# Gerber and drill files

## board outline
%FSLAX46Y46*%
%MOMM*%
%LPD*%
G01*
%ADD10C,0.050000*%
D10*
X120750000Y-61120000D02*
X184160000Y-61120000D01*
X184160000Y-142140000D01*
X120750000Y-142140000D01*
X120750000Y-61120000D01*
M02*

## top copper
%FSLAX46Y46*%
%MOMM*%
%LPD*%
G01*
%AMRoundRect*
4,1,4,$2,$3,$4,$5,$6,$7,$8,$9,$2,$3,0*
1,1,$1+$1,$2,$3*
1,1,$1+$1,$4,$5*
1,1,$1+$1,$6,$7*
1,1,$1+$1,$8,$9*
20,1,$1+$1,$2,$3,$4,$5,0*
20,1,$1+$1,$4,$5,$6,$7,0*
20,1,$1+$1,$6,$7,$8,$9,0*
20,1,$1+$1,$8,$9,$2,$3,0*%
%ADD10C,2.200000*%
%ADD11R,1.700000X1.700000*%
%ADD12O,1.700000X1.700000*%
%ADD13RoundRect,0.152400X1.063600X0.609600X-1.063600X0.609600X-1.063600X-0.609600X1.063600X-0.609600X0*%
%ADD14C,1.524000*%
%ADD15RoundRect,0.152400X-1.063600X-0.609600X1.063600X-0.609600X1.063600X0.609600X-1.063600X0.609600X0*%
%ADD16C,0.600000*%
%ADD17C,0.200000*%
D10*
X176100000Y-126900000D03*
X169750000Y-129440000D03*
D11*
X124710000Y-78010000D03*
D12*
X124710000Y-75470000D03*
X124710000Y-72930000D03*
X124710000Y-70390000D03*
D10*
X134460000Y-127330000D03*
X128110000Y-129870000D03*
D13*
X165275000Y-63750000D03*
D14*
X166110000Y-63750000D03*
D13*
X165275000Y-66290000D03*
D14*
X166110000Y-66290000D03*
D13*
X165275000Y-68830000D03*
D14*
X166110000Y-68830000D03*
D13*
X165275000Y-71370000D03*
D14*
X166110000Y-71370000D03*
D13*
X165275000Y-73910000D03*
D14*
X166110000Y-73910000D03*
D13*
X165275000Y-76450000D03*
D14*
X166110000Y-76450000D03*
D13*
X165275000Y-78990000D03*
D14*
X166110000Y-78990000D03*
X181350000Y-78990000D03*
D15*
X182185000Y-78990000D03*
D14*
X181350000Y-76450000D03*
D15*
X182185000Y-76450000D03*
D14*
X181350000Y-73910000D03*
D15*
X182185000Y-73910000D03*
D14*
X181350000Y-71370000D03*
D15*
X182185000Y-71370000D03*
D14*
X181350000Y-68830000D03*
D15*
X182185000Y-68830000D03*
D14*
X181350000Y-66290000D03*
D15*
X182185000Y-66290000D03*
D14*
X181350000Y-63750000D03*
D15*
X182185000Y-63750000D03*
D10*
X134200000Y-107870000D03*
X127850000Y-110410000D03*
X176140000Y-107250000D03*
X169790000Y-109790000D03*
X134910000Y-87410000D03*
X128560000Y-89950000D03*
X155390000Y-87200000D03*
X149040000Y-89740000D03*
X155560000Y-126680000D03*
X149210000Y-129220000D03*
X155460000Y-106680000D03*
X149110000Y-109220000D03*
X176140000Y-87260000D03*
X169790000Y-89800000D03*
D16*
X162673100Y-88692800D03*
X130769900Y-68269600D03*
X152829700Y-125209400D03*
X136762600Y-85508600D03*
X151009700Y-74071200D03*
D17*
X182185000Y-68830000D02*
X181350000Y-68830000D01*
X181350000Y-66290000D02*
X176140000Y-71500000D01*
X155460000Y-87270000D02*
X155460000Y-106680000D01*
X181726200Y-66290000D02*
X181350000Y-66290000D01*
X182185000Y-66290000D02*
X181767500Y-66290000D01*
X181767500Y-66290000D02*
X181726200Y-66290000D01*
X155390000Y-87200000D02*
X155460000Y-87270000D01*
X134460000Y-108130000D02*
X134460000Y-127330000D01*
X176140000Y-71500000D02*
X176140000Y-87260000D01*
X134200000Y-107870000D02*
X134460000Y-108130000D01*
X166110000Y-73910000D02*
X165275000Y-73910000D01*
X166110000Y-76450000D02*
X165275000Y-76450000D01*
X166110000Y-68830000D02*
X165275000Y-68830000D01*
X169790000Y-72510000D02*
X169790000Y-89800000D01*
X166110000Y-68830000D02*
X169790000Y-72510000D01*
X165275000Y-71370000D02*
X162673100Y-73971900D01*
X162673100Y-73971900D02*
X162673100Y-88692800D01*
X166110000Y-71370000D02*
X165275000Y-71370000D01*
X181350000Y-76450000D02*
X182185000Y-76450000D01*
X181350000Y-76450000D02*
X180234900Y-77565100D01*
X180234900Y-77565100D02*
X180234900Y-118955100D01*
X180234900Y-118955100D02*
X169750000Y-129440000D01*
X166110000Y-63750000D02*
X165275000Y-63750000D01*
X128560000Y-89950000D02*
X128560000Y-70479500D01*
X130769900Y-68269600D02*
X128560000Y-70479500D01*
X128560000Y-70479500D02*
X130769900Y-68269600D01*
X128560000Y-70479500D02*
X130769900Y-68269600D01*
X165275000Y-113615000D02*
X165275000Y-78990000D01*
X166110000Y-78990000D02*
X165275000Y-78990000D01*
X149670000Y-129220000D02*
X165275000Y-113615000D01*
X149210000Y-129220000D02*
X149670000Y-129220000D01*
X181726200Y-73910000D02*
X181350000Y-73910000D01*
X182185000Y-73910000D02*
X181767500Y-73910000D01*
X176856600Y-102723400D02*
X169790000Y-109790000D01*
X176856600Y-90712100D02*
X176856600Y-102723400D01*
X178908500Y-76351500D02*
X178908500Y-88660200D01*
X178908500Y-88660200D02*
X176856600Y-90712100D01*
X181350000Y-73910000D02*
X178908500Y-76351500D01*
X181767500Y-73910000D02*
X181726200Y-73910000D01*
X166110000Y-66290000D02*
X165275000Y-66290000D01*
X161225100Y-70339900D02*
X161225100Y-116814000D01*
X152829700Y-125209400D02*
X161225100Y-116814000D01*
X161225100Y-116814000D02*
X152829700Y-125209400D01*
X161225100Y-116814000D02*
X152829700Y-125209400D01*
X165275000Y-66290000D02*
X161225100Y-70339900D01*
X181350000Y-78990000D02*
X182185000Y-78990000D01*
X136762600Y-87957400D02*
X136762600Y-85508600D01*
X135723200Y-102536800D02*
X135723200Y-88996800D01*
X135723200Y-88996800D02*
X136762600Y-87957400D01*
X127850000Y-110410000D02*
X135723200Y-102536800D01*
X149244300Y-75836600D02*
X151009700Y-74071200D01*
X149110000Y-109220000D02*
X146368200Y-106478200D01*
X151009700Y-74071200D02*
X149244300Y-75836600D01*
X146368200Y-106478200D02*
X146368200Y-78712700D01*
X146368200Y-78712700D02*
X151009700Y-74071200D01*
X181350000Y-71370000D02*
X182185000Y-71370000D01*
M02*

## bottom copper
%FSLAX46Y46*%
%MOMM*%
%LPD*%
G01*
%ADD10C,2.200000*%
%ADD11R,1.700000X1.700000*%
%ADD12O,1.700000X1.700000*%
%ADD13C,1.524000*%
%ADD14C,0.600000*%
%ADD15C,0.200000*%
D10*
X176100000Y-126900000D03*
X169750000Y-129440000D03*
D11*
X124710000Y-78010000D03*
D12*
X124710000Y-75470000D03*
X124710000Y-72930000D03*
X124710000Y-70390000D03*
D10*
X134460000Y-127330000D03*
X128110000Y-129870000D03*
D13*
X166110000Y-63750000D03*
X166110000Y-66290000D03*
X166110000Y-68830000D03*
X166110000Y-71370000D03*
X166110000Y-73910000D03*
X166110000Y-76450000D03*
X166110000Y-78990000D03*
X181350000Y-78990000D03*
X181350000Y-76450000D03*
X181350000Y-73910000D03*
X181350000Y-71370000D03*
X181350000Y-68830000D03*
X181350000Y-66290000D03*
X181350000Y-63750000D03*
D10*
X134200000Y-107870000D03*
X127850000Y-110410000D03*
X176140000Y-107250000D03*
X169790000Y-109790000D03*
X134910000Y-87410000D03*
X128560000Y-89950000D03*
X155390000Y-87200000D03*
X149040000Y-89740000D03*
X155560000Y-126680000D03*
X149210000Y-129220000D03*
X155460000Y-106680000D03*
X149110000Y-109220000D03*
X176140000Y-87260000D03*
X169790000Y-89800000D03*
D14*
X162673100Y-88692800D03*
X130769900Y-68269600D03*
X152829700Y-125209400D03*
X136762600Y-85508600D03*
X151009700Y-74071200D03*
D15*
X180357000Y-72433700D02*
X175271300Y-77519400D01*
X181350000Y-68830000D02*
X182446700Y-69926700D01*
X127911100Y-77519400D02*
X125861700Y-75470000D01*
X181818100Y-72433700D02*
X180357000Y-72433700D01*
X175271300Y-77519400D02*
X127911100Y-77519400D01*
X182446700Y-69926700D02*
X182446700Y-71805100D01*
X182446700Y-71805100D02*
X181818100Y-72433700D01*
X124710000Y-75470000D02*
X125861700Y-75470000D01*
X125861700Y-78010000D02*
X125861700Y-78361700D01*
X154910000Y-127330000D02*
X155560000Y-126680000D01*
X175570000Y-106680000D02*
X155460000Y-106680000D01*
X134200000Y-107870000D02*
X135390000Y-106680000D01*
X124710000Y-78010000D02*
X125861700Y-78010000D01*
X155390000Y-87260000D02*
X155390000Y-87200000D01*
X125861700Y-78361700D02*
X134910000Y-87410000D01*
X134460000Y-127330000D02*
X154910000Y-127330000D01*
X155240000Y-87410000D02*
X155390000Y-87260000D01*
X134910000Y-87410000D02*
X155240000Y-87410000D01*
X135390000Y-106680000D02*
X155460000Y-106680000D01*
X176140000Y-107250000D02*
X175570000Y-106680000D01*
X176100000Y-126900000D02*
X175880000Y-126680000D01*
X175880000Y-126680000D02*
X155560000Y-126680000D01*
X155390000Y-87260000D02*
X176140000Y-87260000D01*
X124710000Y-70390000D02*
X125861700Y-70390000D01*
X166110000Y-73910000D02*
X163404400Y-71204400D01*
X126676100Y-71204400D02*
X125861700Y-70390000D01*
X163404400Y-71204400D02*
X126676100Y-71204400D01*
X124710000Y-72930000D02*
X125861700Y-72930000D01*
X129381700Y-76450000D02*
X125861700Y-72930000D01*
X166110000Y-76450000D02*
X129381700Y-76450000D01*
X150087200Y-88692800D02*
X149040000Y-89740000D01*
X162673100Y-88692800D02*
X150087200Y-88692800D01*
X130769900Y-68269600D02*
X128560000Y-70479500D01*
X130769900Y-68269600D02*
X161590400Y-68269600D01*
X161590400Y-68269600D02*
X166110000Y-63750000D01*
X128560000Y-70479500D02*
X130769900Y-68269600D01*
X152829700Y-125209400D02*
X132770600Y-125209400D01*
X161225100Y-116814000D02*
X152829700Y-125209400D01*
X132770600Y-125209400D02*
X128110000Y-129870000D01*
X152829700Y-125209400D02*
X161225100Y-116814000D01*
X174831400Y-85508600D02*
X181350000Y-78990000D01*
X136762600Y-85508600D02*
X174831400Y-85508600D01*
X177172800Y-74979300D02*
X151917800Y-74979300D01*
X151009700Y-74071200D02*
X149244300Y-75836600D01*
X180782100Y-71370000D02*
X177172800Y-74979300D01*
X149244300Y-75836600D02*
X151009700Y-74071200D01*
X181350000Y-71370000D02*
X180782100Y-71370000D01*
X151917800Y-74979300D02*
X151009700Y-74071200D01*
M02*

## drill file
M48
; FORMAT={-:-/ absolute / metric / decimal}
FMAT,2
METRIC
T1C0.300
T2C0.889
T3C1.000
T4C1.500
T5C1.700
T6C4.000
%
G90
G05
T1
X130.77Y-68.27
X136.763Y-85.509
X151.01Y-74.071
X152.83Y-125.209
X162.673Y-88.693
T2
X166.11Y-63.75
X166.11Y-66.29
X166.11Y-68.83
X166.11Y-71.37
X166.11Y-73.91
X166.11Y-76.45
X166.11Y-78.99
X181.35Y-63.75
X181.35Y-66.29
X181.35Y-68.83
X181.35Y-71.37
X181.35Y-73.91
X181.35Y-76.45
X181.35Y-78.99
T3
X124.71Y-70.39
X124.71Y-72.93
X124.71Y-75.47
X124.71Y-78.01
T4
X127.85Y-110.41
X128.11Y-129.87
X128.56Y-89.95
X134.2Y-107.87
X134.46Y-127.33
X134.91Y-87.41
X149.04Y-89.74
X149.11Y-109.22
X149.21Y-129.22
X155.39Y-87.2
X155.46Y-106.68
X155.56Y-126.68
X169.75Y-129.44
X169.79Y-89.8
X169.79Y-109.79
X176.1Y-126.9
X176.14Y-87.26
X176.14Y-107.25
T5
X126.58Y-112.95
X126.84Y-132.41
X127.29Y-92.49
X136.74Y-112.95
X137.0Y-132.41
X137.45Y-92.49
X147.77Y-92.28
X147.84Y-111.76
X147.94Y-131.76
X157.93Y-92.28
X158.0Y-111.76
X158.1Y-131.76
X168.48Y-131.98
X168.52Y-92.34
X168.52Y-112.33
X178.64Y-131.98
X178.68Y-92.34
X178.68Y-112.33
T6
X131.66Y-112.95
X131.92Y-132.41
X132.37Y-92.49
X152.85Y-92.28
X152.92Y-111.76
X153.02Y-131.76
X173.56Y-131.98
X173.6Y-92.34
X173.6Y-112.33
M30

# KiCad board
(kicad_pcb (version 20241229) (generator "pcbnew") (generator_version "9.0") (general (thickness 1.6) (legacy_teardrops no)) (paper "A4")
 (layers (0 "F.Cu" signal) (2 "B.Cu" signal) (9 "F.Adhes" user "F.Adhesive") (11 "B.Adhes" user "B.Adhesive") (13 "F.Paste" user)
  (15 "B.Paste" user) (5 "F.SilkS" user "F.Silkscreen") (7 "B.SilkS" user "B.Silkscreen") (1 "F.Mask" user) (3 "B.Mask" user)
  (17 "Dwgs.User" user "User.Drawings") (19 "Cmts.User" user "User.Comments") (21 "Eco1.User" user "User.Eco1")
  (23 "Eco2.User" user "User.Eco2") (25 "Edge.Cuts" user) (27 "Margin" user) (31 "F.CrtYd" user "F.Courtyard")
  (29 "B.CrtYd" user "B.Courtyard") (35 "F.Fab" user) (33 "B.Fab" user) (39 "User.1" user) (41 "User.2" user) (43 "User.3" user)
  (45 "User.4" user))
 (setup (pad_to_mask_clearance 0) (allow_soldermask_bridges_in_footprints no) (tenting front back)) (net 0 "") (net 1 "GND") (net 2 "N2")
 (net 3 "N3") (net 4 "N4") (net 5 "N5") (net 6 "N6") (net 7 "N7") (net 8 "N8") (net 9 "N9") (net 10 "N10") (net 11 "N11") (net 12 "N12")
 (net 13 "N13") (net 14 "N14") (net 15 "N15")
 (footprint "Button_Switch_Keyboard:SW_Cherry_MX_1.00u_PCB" (layer "F.Cu") (at 176.1 126.9)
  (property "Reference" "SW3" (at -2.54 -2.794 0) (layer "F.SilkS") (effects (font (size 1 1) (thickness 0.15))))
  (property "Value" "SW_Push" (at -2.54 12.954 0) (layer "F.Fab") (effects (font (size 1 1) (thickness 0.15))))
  (pad "" np_thru_hole circle (at -7.62 5.08) (size 1.7 1.7) (drill 1.7) (layers "*.Cu" "*.Mask"))
  (pad "" np_thru_hole circle (at -2.54 5.08) (size 4 4) (drill 4) (layers "*.Cu" "*.Mask"))
  (pad "" np_thru_hole circle (at 2.54 5.08) (size 1.7 1.7) (drill 1.7) (layers "*.Cu" "*.Mask"))
  (pad "1" thru_hole circle (at 0 0) (size 2.2 2.2) (drill 1.5) (layers "*.Cu" "*.Mask") (remove_unused_layers no) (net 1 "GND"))
  (pad "2" thru_hole circle (at -6.35 2.54) (size 2.2 2.2) (drill 1.5) (layers "*.Cu" "*.Mask") (remove_unused_layers no) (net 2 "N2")))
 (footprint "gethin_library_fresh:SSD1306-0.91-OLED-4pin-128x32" (layer "F.Cu") (at 161.21 80.2 180)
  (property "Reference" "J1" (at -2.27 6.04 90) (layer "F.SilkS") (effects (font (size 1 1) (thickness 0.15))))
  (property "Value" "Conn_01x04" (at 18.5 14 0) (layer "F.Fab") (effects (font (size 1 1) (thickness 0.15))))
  (pad "1" thru_hole rect (at 36.5 2.19 180) (size 1.7 1.7) (drill 1) (layers "*.Cu" "*.Mask") (remove_unused_layers no) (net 1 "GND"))
  (pad "2" thru_hole oval (at 36.5 4.73 180) (size 1.7 1.7) (drill 1) (layers "*.Cu" "*.Mask") (remove_unused_layers no) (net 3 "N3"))
  (pad "3" thru_hole oval (at 36.5 7.27 180) (size 1.7 1.7) (drill 1) (layers "*.Cu" "*.Mask") (remove_unused_layers no) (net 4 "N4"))
  (pad "4" thru_hole oval (at 36.5 9.81 180) (size 1.7 1.7) (drill 1) (layers "*.Cu" "*.Mask") (remove_unused_layers no) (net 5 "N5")))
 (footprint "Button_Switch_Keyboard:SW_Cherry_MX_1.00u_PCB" (layer "F.Cu") (at 134.46 127.33)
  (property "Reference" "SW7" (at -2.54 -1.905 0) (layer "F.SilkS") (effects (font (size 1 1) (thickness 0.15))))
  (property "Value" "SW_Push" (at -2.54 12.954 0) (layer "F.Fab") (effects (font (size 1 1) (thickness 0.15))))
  (pad "" np_thru_hole circle (at -7.62 5.08) (size 1.7 1.7) (drill 1.7) (layers "*.Cu" "*.Mask"))
  (pad "" np_thru_hole circle (at -2.54 5.08) (size 4 4) (drill 4) (layers "*.Cu" "*.Mask"))
  (pad "" np_thru_hole circle (at 2.54 5.08) (size 1.7 1.7) (drill 1.7) (layers "*.Cu" "*.Mask"))
  (pad "1" thru_hole circle (at 0 0) (size 2.2 2.2) (drill 1.5) (layers "*.Cu" "*.Mask") (remove_unused_layers no) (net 1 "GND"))
  (pad "2" thru_hole circle (at -6.35 2.54) (size 2.2 2.2) (drill 1.5) (layers "*.Cu" "*.Mask") (remove_unused_layers no) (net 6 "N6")))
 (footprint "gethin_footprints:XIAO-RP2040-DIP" (layer "F.Cu") (at 173.73 71.37)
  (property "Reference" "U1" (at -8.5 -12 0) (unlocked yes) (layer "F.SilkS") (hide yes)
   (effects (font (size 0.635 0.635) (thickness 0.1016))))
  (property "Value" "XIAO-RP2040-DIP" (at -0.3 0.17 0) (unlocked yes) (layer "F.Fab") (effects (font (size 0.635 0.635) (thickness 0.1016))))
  (pad "1" smd roundrect (at -8.455 -7.62 180) (size 2.432 1.524) (layers "F.Cu" "F.Mask") (roundrect_rratio 0.1) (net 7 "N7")
   (thermal_bridge_angle 45))
  (pad "1" thru_hole circle (at -7.62 -7.62 180) (size 1.524 1.524) (drill 0.889) (layers "*.Cu" "*.Mask") (remove_unused_layers no)
   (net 7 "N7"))
  (pad "2" smd roundrect (at -8.455 -5.08 180) (size 2.432 1.524) (layers "F.Cu" "F.Mask") (roundrect_rratio 0.1) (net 6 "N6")
   (thermal_bridge_angle 45))
  (pad "2" thru_hole circle (at -7.62 -5.08 180) (size 1.524 1.524) (drill 0.889) (layers "*.Cu" "*.Mask") (remove_unused_layers no)
   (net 6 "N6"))
  (pad "3" smd roundrect (at -8.455 -2.54 180) (size 2.432 1.524) (layers "F.Cu" "F.Mask") (roundrect_rratio 0.1) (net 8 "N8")
   (thermal_bridge_angle 45))
  (pad "3" thru_hole circle (at -7.62 -2.54 180) (size 1.524 1.524) (drill 0.889) (layers "*.Cu" "*.Mask") (remove_unused_layers no)
   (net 8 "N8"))
  (pad "4" smd roundrect (at -8.455 0 180) (size 2.432 1.524) (layers "F.Cu" "F.Mask") (roundrect_rratio 0.1) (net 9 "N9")
   (thermal_bridge_angle 45))
  (pad "4" thru_hole circle (at -7.62 0 180) (size 1.524 1.524) (drill 0.889) (layers "*.Cu" "*.Mask") (remove_unused_layers no)
   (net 9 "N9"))
  (pad "5" smd roundrect (at -8.455 2.54 180) (size 2.432 1.524) (layers "F.Cu" "F.Mask") (roundrect_rratio 0.1) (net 5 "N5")
   (thermal_bridge_angle 45))
  (pad "5" thru_hole circle (at -7.62 2.54 180) (size 1.524 1.524) (drill 0.889) (layers "*.Cu" "*.Mask") (remove_unused_layers no)
   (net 5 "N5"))
  (pad "6" smd roundrect (at -8.455 5.08 180) (size 2.432 1.524) (layers "F.Cu" "F.Mask") (roundrect_rratio 0.1) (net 4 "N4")
   (thermal_bridge_angle 45))
  (pad "6" thru_hole circle (at -7.62 5.08 180) (size 1.524 1.524) (drill 0.889) (layers "*.Cu" "*.Mask") (remove_unused_layers no)
   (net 4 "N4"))
  (pad "7" smd roundrect (at -8.455 7.62 180) (size 2.432 1.524) (layers "F.Cu" "F.Mask") (roundrect_rratio 0.1) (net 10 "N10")
   (thermal_bridge_angle 45))
  (pad "7" thru_hole circle (at -7.62 7.62 180) (size 1.524 1.524) (drill 0.889) (layers "*.Cu" "*.Mask") (remove_unused_layers no)
   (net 10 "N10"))
  (pad "8" thru_hole circle (at 7.62 7.62) (size 1.524 1.524) (drill 0.889) (layers "*.Cu" "*.Mask") (remove_unused_layers no)
   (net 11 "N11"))
  (pad "8" smd roundrect (at 8.455 7.62) (size 2.432 1.524) (layers "F.Cu" "F.Mask") (roundrect_rratio 0.1) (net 11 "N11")
   (thermal_bridge_angle 45))
  (pad "9" thru_hole circle (at 7.62 5.08) (size 1.524 1.524) (drill 0.889) (layers "*.Cu" "*.Mask") (remove_unused_layers no) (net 2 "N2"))
  (pad "9" smd roundrect (at 8.455 5.08) (size 2.432 1.524) (layers "F.Cu" "F.Mask") (roundrect_rratio 0.1) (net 2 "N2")
   (thermal_bridge_angle 45))
  (pad "10" thru_hole circle (at 7.62 2.54) (size 1.524 1.524) (drill 0.889) (layers "*.Cu" "*.Mask") (remove_unused_layers no)
   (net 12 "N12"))
  (pad "10" smd roundrect (at 8.455 2.54) (size 2.432 1.524) (layers "F.Cu" "F.Mask") (roundrect_rratio 0.1) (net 12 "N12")
   (thermal_bridge_angle 45))
  (pad "11" thru_hole circle (at 7.62 0) (size 1.524 1.524) (drill 0.889) (layers "*.Cu" "*.Mask") (remove_unused_layers no) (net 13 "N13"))
  (pad "11" smd roundrect (at 8.455 0) (size 2.432 1.524) (layers "F.Cu" "F.Mask") (roundrect_rratio 0.1) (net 13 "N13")
   (thermal_bridge_angle 45))
  (pad "12" thru_hole circle (at 7.62 -2.54) (size 1.524 1.524) (drill 0.889) (layers "*.Cu" "*.Mask") (remove_unused_layers no)
   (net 3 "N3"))
  (pad "12" smd roundrect (at 8.455 -2.54) (size 2.432 1.524) (layers "F.Cu" "F.Mask") (roundrect_rratio 0.1) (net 3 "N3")
   (thermal_bridge_angle 45))
  (pad "13" thru_hole circle (at 7.62 -5.08) (size 1.524 1.524) (drill 0.889) (layers "*.Cu" "*.Mask") (remove_unused_layers no)
   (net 1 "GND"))
  (pad "13" smd roundrect (at 8.455 -5.08) (size 2.432 1.524) (layers "F.Cu" "F.Mask") (roundrect_rratio 0.1) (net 1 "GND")
   (thermal_bridge_angle 45))
  (pad "14" thru_hole circle (at 7.62 -7.62) (size 1.524 1.524) (drill 0.889) (layers "*.Cu" "*.Mask") (remove_unused_layers no)
   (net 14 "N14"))
  (pad "14" smd roundrect (at 8.455 -7.62) (size 2.432 1.524) (layers "F.Cu" "F.Mask") (roundrect_rratio 0.1) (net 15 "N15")
   (thermal_bridge_angle 45)))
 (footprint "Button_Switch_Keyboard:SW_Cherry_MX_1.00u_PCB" (layer "F.Cu") (at 134.2 107.87)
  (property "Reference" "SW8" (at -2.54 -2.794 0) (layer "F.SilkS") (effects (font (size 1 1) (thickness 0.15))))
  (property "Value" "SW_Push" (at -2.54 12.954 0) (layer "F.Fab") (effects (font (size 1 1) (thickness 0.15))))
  (pad "" np_thru_hole circle (at -7.62 5.08) (size 1.7 1.7) (drill 1.7) (layers "*.Cu" "*.Mask"))
  (pad "" np_thru_hole circle (at -2.54 5.08) (size 4 4) (drill 4) (layers "*.Cu" "*.Mask"))
  (pad "" np_thru_hole circle (at 2.54 5.08) (size 1.7 1.7) (drill 1.7) (layers "*.Cu" "*.Mask"))
  (pad "1" thru_hole circle (at 0 0) (size 2.2 2.2) (drill 1.5) (layers "*.Cu" "*.Mask") (remove_unused_layers no) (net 1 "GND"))
  (pad "2" thru_hole circle (at -6.35 2.54) (size 2.2 2.2) (drill 1.5) (layers "*.Cu" "*.Mask") (remove_unused_layers no) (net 11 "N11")))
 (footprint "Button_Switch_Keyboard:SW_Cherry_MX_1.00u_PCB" (layer "F.Cu") (at 176.14 107.25)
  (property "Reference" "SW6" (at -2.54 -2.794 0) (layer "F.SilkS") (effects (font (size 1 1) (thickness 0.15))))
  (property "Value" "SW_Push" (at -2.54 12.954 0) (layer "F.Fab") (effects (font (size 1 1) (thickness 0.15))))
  (pad "" np_thru_hole circle (at -7.62 5.08) (size 1.7 1.7) (drill 1.7) (layers "*.Cu" "*.Mask"))
  (pad "" np_thru_hole circle (at -2.54 5.08) (size 4 4) (drill 4) (layers "*.Cu" "*.Mask"))
  (pad "" np_thru_hole circle (at 2.54 5.08) (size 1.7 1.7) (drill 1.7) (layers "*.Cu" "*.Mask"))
  (pad "1" thru_hole circle (at 0 0) (size 2.2 2.2) (drill 1.5) (layers "*.Cu" "*.Mask") (remove_unused_layers no) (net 1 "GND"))
  (pad "2" thru_hole circle (at -6.35 2.54) (size 2.2 2.2) (drill 1.5) (layers "*.Cu" "*.Mask") (remove_unused_layers no) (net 12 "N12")))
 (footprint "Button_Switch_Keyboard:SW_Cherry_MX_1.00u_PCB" (layer "F.Cu") (at 134.91 87.41)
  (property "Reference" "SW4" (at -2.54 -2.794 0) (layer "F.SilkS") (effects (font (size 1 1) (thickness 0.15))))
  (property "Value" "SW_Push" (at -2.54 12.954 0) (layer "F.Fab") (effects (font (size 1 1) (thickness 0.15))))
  (pad "" np_thru_hole circle (at -7.62 5.08) (size 1.7 1.7) (drill 1.7) (layers "*.Cu" "*.Mask"))
  (pad "" np_thru_hole circle (at -2.54 5.08) (size 4 4) (drill 4) (layers "*.Cu" "*.Mask"))
  (pad "" np_thru_hole circle (at 2.54 5.08) (size 1.7 1.7) (drill 1.7) (layers "*.Cu" "*.Mask"))
  (pad "1" thru_hole circle (at 0 0) (size 2.2 2.2) (drill 1.5) (layers "*.Cu" "*.Mask") (remove_unused_layers no) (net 1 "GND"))
  (pad "2" thru_hole circle (at -6.35 2.54) (size 2.2 2.2) (drill 1.5) (layers "*.Cu" "*.Mask") (remove_unused_layers no) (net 7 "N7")))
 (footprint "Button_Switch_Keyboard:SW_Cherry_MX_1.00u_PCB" (layer "F.Cu") (at 155.39 87.2)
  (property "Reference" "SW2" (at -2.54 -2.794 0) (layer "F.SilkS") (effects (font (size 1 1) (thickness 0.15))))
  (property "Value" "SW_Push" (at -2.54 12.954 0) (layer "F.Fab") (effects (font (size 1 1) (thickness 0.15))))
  (pad "" np_thru_hole circle (at -7.62 5.08) (size 1.7 1.7) (drill 1.7) (layers "*.Cu" "*.Mask"))
  (pad "" np_thru_hole circle (at -2.54 5.08) (size 4 4) (drill 4) (layers "*.Cu" "*.Mask"))
  (pad "" np_thru_hole circle (at 2.54 5.08) (size 1.7 1.7) (drill 1.7) (layers "*.Cu" "*.Mask"))
  (pad "1" thru_hole circle (at 0 0) (size 2.2 2.2) (drill 1.5) (layers "*.Cu" "*.Mask") (remove_unused_layers no) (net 1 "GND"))
  (pad "2" thru_hole circle (at -6.35 2.54) (size 2.2 2.2) (drill 1.5) (layers "*.Cu" "*.Mask") (remove_unused_layers no) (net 9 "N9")))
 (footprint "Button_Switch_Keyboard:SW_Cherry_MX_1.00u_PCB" (layer "F.Cu") (at 155.56 126.68)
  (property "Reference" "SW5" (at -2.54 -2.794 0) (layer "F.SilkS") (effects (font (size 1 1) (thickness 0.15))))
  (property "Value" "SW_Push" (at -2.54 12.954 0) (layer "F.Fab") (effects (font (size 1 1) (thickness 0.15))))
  (pad "" np_thru_hole circle (at -7.62 5.08) (size 1.7 1.7) (drill 1.7) (layers "*.Cu" "*.Mask"))
  (pad "" np_thru_hole circle (at -2.54 5.08) (size 4 4) (drill 4) (layers "*.Cu" "*.Mask"))
  (pad "" np_thru_hole circle (at 2.54 5.08) (size 1.7 1.7) (drill 1.7) (layers "*.Cu" "*.Mask"))
  (pad "1" thru_hole circle (at 0 0) (size 2.2 2.2) (drill 1.5) (layers "*.Cu" "*.Mask") (remove_unused_layers no) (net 1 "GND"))
  (pad "2" thru_hole circle (at -6.35 2.54) (size 2.2 2.2) (drill 1.5) (layers "*.Cu" "*.Mask") (remove_unused_layers no) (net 10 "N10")))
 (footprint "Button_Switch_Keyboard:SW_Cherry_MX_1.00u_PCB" (layer "F.Cu") (at 155.46 106.68)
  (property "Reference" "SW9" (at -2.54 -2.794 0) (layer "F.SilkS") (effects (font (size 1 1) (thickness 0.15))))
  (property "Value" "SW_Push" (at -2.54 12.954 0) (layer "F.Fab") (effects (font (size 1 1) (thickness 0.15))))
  (pad "" np_thru_hole circle (at -7.62 5.08) (size 1.7 1.7) (drill 1.7) (layers "*.Cu" "*.Mask"))
  (pad "" np_thru_hole circle (at -2.54 5.08) (size 4 4) (drill 4) (layers "*.Cu" "*.Mask"))
  (pad "" np_thru_hole circle (at 2.54 5.08) (size 1.7 1.7) (drill 1.7) (layers "*.Cu" "*.Mask"))
  (pad "1" thru_hole circle (at 0 0) (size 2.2 2.2) (drill 1.5) (layers "*.Cu" "*.Mask") (remove_unused_layers no) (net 1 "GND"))
  (pad "2" thru_hole circle (at -6.35 2.54) (size 2.2 2.2) (drill 1.5) (layers "*.Cu" "*.Mask") (remove_unused_layers no) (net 13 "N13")))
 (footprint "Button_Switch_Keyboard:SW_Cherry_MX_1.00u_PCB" (layer "F.Cu") (at 176.14 87.26)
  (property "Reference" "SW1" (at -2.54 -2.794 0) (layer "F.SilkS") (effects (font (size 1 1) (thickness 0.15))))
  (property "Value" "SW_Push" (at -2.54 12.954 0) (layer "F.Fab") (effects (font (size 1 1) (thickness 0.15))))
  (pad "" np_thru_hole circle (at -7.62 5.08) (size 1.7 1.7) (drill 1.7) (layers "*.Cu" "*.Mask"))
  (pad "" np_thru_hole circle (at -2.54 5.08) (size 4 4) (drill 4) (layers "*.Cu" "*.Mask"))
  (pad "" np_thru_hole circle (at 2.54 5.08) (size 1.7 1.7) (drill 1.7) (layers "*.Cu" "*.Mask"))
  (pad "1" thru_hole circle (at 0 0) (size 2.2 2.2) (drill 1.5) (layers "*.Cu" "*.Mask") (remove_unused_layers no) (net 1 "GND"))
  (pad "2" thru_hole circle (at -6.35 2.54) (size 2.2 2.2) (drill 1.5) (layers "*.Cu" "*.Mask") (remove_unused_layers no) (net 8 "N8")))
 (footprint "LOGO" (layer "B.Cu") (at 141.611711 75.169904 180)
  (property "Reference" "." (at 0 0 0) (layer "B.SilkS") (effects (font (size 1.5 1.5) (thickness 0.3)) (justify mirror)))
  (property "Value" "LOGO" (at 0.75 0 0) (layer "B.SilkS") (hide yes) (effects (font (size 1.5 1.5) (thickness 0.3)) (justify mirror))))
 (gr_rect (start 120.75 61.12) (end 184.16 142.14) (stroke (width 0.05) (type default)) (fill no) (layer "Edge.Cuts"))
 (segment (start 182.185 68.83) (end 181.35 68.83) (width 0.2) (layer "F.Cu") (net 3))
 (segment (start 180.357 72.4337) (end 175.2713 77.5194) (width 0.2) (layer "B.Cu") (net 3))
 (segment (start 181.35 68.83) (end 182.4467 69.9267) (width 0.2) (layer "B.Cu") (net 3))
 (segment (start 127.9111 77.5194) (end 125.8617 75.47) (width 0.2) (layer "B.Cu") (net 3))
 (segment (start 181.8181 72.4337) (end 180.357 72.4337) (width 0.2) (layer "B.Cu") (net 3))
 (segment (start 175.2713 77.5194) (end 127.9111 77.5194) (width 0.2) (layer "B.Cu") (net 3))
 (segment (start 182.4467 69.9267) (end 182.4467 71.8051) (width 0.2) (layer "B.Cu") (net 3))
 (segment (start 182.4467 71.8051) (end 181.8181 72.4337) (width 0.2) (layer "B.Cu") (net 3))
 (segment (start 124.71 75.47) (end 125.8617 75.47) (width 0.2) (layer "B.Cu") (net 3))
 (segment (start 181.35 66.29) (end 176.14 71.5) (width 0.2) (layer "F.Cu") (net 1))
 (segment (start 155.46 87.27) (end 155.46 106.68) (width 0.2) (layer "F.Cu") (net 1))
 (segment (start 181.7262 66.29) (end 181.35 66.29) (width 0.2) (layer "F.Cu") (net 1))
 (segment (start 182.185 66.29) (end 181.7675 66.29) (width 0.2) (layer "F.Cu") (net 1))
 (segment (start 181.7675 66.29) (end 181.7262 66.29) (width 0.2) (layer "F.Cu") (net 1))
 (segment (start 155.39 87.2) (end 155.46 87.27) (width 0.2) (layer "F.Cu") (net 1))
 (segment (start 134.46 108.13) (end 134.46 127.33) (width 0.2) (layer "F.Cu") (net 1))
 (segment (start 176.14 71.5) (end 176.14 87.26) (width 0.2) (layer "F.Cu") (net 1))
 (segment (start 134.2 107.87) (end 134.46 108.13) (width 0.2) (layer "F.Cu") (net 1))
 (segment (start 125.8617 78.01) (end 125.8617 78.3617) (width 0.2) (layer "B.Cu") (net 1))
 (segment (start 154.91 127.33) (end 155.56 126.68) (width 0.2) (layer "B.Cu") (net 1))
 (segment (start 175.57 106.68) (end 155.46 106.68) (width 0.2) (layer "B.Cu") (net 1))
 (segment (start 134.2 107.87) (end 135.39 106.68) (width 0.2) (layer "B.Cu") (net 1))
 (segment (start 124.71 78.01) (end 125.8617 78.01) (width 0.2) (layer "B.Cu") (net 1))
 (segment (start 155.39 87.26) (end 155.39 87.2) (width 0.2) (layer "B.Cu") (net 1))
 (segment (start 125.8617 78.3617) (end 134.91 87.41) (width 0.2) (layer "B.Cu") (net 1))
 (segment (start 134.46 127.33) (end 154.91 127.33) (width 0.2) (layer "B.Cu") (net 1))
 (segment (start 155.24 87.41) (end 155.39 87.26) (width 0.2) (layer "B.Cu") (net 1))
 (segment (start 134.91 87.41) (end 155.24 87.41) (width 0.2) (layer "B.Cu") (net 1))
 (segment (start 135.39 106.68) (end 155.46 106.68) (width 0.2) (layer "B.Cu") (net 1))
 (segment (start 176.14 107.25) (end 175.57 106.68) (width 0.2) (layer "B.Cu") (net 1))
 (segment (start 176.1 126.9) (end 175.88 126.68) (width 0.2) (layer "B.Cu") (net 1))
 (segment (start 175.88 126.68) (end 155.56 126.68) (width 0.2) (layer "B.Cu") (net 1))
 (segment (start 155.39 87.26) (end 176.14 87.26) (width 0.2) (layer "B.Cu") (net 1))
 (segment (start 166.11 73.91) (end 165.275 73.91) (width 0.2) (layer "F.Cu") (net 5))
 (segment (start 124.71 70.39) (end 125.8617 70.39) (width 0.2) (layer "B.Cu") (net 5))
 (segment (start 166.11 73.91) (end 163.4044 71.2044) (width 0.2) (layer "B.Cu") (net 5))
 (segment (start 126.6761 71.2044) (end 125.8617 70.39) (width 0.2) (layer "B.Cu") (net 5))
 (segment (start 163.4044 71.2044) (end 126.6761 71.2044) (width 0.2) (layer "B.Cu") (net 5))
 (segment (start 166.11 76.45) (end 165.275 76.45) (width 0.2) (layer "F.Cu") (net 4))
 (segment (start 124.71 72.93) (end 125.8617 72.93) (width 0.2) (layer "B.Cu") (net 4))
 (segment (start 129.3817 76.45) (end 125.8617 72.93) (width 0.2) (layer "B.Cu") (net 4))
 (segment (start 166.11 76.45) (end 129.3817 76.45) (width 0.2) (layer "B.Cu") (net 4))
 (segment (start 166.11 68.83) (end 165.275 68.83) (width 0.2) (layer "F.Cu") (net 8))
 (segment (start 169.79 72.51) (end 169.79 89.8) (width 0.2) (layer "F.Cu") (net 8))
 (segment (start 166.11 68.83) (end 169.79 72.51) (width 0.2) (layer "F.Cu") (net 8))
 (segment (start 165.275 71.37) (end 162.6731 73.9719) (width 0.2) (layer "F.Cu") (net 9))
 (segment (start 162.6731 73.9719) (end 162.6731 88.6928) (width 0.2) (layer "F.Cu") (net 9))
 (segment (start 166.11 71.37) (end 165.275 71.37) (width 0.2) (layer "F.Cu") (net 9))
 (via (at 162.6731 88.6928) (size 0.6) (drill 0.3) (layers "F.Cu" "B.Cu") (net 9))
 (segment (start 150.0872 88.6928) (end 149.04 89.74) (width 0.2) (layer "B.Cu") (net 9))
 (segment (start 162.6731 88.6928) (end 150.0872 88.6928) (width 0.2) (layer "B.Cu") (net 9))
 (segment (start 181.35 76.45) (end 182.185 76.45) (width 0.2) (layer "F.Cu") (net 2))
 (segment (start 181.35 76.45) (end 180.2349 77.5651) (width 0.2) (layer "F.Cu") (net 2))
 (segment (start 180.2349 77.5651) (end 180.2349 118.9551) (width 0.2) (layer "F.Cu") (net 2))
 (segment (start 180.2349 118.9551) (end 169.75 129.44) (width 0.2) (layer "F.Cu") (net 2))
 (segment (start 166.11 63.75) (end 165.275 63.75) (width 0.2) (layer "F.Cu") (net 7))
 (segment (start 128.56 89.95) (end 128.56 70.4795) (width 0.2) (layer "F.Cu") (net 7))
 (segment (start 130.7699 68.2696) (end 128.56 70.4795) (width 0.2) (layer "F.Cu") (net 7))
 (segment (start 128.56 70.4795) (end 130.7699 68.2696) (width 0.2) (layer "F.Cu") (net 7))
 (segment (start 128.56 70.4795) (end 130.7699 68.2696) (width 0.2) (layer "F.Cu") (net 7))
 (via (at 130.7699 68.2696) (size 0.6) (drill 0.3) (layers "F.Cu" "B.Cu") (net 7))
 (segment (start 130.7699 68.2696) (end 128.56 70.4795) (width 0.2) (layer "B.Cu") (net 7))
 (segment (start 130.7699 68.2696) (end 161.5904 68.2696) (width 0.2) (layer "B.Cu") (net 7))
 (segment (start 161.5904 68.2696) (end 166.11 63.75) (width 0.2) (layer "B.Cu") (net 7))
 (segment (start 128.56 70.4795) (end 130.7699 68.2696) (width 0.2) (layer "B.Cu") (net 7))
 (segment (start 165.275 113.615) (end 165.275 78.99) (width 0.2) (layer "F.Cu") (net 10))
 (segment (start 166.11 78.99) (end 165.275 78.99) (width 0.2) (layer "F.Cu") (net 10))
 (segment (start 149.67 129.22) (end 165.275 113.615) (width 0.2) (layer "F.Cu") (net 10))
 (segment (start 149.21 129.22) (end 149.67 129.22) (width 0.2) (layer "F.Cu") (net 10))
 (segment (start 181.7262 73.91) (end 181.35 73.91) (width 0.2) (layer "F.Cu") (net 12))
 (segment (start 182.185 73.91) (end 181.7675 73.91) (width 0.2) (layer "F.Cu") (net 12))
 (segment (start 176.8566 102.7234) (end 169.79 109.79) (width 0.2) (layer "F.Cu") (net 12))
 (segment (start 176.8566 90.7121) (end 176.8566 102.7234) (width 0.2) (layer "F.Cu") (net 12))
 (segment (start 178.9085 76.3515) (end 178.9085 88.6602) (width 0.2) (layer "F.Cu") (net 12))
 (segment (start 178.9085 88.6602) (end 176.8566 90.7121) (width 0.2) (layer "F.Cu") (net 12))
 (segment (start 181.35 73.91) (end 178.9085 76.3515) (width 0.2) (layer "F.Cu") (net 12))
 (segment (start 181.7675 73.91) (end 181.7262 73.91) (width 0.2) (layer "F.Cu") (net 12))
 (segment (start 166.11 66.29) (end 165.275 66.29) (width 0.2) (layer "F.Cu") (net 6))
 (segment (start 161.2251 70.3399) (end 161.2251 116.814) (width 0.2) (layer "F.Cu") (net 6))
 (segment (start 152.8297 125.2094) (end 161.2251 116.814) (width 0.2) (layer "F.Cu") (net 6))
 (segment (start 161.2251 116.814) (end 152.8297 125.2094) (width 0.2) (layer "F.Cu") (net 6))
 (segment (start 161.2251 116.814) (end 152.8297 125.2094) (width 0.2) (layer "F.Cu") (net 6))
 (segment (start 165.275 66.29) (end 161.2251 70.3399) (width 0.2) (layer "F.Cu") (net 6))
 (via (at 152.8297 125.2094) (size 0.6) (drill 0.3) (layers "F.Cu" "B.Cu") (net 6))
 (segment (start 152.8297 125.2094) (end 132.7706 125.2094) (width 0.2) (layer "B.Cu") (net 6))
 (segment (start 161.2251 116.814) (end 152.8297 125.2094) (width 0.2) (layer "B.Cu") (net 6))
 (segment (start 132.7706 125.2094) (end 128.11 129.87) (width 0.2) (layer "B.Cu") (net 6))
 (segment (start 152.8297 125.2094) (end 161.2251 116.814) (width 0.2) (layer "B.Cu") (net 6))
 (segment (start 181.35 78.99) (end 182.185 78.99) (width 0.2) (layer "F.Cu") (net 11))
 (segment (start 136.7626 87.9574) (end 136.7626 85.5086) (width 0.2) (layer "F.Cu") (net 11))
 (segment (start 135.7232 102.5368) (end 135.7232 88.9968) (width 0.2) (layer "F.Cu") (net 11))
 (segment (start 135.7232 88.9968) (end 136.7626 87.9574) (width 0.2) (layer "F.Cu") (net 11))
 (segment (start 127.85 110.41) (end 135.7232 102.5368) (width 0.2) (layer "F.Cu") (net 11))
 (via (at 136.7626 85.5086) (size 0.6) (drill 0.3) (layers "F.Cu" "B.Cu") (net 11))
 (segment (start 174.8314 85.5086) (end 181.35 78.99) (width 0.2) (layer "B.Cu") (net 11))
 (segment (start 136.7626 85.5086) (end 174.8314 85.5086) (width 0.2) (layer "B.Cu") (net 11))
 (segment (start 149.2443 75.8366) (end 151.0097 74.0712) (width 0.2) (layer "F.Cu") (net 13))
 (segment (start 149.11 109.22) (end 146.3682 106.4782) (width 0.2) (layer "F.Cu") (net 13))
 (segment (start 151.0097 74.0712) (end 149.2443 75.8366) (width 0.2) (layer "F.Cu") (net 13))
 (segment (start 146.3682 106.4782) (end 146.3682 78.7127) (width 0.2) (layer "F.Cu") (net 13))
 (segment (start 146.3682 78.7127) (end 151.0097 74.0712) (width 0.2) (layer "F.Cu") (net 13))
 (segment (start 181.35 71.37) (end 182.185 71.37) (width 0.2) (layer "F.Cu") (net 13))
 (via (at 151.0097 74.0712) (size 0.6) (drill 0.3) (layers "F.Cu" "B.Cu") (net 13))
 (segment (start 177.1728 74.9793) (end 151.9178 74.9793) (width 0.2) (layer "B.Cu") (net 13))
 (segment (start 151.0097 74.0712) (end 149.2443 75.8366) (width 0.2) (layer "B.Cu") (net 13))
 (segment (start 180.7821 71.37) (end 177.1728 74.9793) (width 0.2) (layer "B.Cu") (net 13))
 (segment (start 149.2443 75.8366) (end 151.0097 74.0712) (width 0.2) (layer "B.Cu") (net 13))
 (segment (start 181.35 71.37) (end 180.7821 71.37) (width 0.2) (layer "B.Cu") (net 13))
 (segment (start 151.9178 74.9793) (end 151.0097 74.0712) (width 0.2) (layer "B.Cu") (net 13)))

